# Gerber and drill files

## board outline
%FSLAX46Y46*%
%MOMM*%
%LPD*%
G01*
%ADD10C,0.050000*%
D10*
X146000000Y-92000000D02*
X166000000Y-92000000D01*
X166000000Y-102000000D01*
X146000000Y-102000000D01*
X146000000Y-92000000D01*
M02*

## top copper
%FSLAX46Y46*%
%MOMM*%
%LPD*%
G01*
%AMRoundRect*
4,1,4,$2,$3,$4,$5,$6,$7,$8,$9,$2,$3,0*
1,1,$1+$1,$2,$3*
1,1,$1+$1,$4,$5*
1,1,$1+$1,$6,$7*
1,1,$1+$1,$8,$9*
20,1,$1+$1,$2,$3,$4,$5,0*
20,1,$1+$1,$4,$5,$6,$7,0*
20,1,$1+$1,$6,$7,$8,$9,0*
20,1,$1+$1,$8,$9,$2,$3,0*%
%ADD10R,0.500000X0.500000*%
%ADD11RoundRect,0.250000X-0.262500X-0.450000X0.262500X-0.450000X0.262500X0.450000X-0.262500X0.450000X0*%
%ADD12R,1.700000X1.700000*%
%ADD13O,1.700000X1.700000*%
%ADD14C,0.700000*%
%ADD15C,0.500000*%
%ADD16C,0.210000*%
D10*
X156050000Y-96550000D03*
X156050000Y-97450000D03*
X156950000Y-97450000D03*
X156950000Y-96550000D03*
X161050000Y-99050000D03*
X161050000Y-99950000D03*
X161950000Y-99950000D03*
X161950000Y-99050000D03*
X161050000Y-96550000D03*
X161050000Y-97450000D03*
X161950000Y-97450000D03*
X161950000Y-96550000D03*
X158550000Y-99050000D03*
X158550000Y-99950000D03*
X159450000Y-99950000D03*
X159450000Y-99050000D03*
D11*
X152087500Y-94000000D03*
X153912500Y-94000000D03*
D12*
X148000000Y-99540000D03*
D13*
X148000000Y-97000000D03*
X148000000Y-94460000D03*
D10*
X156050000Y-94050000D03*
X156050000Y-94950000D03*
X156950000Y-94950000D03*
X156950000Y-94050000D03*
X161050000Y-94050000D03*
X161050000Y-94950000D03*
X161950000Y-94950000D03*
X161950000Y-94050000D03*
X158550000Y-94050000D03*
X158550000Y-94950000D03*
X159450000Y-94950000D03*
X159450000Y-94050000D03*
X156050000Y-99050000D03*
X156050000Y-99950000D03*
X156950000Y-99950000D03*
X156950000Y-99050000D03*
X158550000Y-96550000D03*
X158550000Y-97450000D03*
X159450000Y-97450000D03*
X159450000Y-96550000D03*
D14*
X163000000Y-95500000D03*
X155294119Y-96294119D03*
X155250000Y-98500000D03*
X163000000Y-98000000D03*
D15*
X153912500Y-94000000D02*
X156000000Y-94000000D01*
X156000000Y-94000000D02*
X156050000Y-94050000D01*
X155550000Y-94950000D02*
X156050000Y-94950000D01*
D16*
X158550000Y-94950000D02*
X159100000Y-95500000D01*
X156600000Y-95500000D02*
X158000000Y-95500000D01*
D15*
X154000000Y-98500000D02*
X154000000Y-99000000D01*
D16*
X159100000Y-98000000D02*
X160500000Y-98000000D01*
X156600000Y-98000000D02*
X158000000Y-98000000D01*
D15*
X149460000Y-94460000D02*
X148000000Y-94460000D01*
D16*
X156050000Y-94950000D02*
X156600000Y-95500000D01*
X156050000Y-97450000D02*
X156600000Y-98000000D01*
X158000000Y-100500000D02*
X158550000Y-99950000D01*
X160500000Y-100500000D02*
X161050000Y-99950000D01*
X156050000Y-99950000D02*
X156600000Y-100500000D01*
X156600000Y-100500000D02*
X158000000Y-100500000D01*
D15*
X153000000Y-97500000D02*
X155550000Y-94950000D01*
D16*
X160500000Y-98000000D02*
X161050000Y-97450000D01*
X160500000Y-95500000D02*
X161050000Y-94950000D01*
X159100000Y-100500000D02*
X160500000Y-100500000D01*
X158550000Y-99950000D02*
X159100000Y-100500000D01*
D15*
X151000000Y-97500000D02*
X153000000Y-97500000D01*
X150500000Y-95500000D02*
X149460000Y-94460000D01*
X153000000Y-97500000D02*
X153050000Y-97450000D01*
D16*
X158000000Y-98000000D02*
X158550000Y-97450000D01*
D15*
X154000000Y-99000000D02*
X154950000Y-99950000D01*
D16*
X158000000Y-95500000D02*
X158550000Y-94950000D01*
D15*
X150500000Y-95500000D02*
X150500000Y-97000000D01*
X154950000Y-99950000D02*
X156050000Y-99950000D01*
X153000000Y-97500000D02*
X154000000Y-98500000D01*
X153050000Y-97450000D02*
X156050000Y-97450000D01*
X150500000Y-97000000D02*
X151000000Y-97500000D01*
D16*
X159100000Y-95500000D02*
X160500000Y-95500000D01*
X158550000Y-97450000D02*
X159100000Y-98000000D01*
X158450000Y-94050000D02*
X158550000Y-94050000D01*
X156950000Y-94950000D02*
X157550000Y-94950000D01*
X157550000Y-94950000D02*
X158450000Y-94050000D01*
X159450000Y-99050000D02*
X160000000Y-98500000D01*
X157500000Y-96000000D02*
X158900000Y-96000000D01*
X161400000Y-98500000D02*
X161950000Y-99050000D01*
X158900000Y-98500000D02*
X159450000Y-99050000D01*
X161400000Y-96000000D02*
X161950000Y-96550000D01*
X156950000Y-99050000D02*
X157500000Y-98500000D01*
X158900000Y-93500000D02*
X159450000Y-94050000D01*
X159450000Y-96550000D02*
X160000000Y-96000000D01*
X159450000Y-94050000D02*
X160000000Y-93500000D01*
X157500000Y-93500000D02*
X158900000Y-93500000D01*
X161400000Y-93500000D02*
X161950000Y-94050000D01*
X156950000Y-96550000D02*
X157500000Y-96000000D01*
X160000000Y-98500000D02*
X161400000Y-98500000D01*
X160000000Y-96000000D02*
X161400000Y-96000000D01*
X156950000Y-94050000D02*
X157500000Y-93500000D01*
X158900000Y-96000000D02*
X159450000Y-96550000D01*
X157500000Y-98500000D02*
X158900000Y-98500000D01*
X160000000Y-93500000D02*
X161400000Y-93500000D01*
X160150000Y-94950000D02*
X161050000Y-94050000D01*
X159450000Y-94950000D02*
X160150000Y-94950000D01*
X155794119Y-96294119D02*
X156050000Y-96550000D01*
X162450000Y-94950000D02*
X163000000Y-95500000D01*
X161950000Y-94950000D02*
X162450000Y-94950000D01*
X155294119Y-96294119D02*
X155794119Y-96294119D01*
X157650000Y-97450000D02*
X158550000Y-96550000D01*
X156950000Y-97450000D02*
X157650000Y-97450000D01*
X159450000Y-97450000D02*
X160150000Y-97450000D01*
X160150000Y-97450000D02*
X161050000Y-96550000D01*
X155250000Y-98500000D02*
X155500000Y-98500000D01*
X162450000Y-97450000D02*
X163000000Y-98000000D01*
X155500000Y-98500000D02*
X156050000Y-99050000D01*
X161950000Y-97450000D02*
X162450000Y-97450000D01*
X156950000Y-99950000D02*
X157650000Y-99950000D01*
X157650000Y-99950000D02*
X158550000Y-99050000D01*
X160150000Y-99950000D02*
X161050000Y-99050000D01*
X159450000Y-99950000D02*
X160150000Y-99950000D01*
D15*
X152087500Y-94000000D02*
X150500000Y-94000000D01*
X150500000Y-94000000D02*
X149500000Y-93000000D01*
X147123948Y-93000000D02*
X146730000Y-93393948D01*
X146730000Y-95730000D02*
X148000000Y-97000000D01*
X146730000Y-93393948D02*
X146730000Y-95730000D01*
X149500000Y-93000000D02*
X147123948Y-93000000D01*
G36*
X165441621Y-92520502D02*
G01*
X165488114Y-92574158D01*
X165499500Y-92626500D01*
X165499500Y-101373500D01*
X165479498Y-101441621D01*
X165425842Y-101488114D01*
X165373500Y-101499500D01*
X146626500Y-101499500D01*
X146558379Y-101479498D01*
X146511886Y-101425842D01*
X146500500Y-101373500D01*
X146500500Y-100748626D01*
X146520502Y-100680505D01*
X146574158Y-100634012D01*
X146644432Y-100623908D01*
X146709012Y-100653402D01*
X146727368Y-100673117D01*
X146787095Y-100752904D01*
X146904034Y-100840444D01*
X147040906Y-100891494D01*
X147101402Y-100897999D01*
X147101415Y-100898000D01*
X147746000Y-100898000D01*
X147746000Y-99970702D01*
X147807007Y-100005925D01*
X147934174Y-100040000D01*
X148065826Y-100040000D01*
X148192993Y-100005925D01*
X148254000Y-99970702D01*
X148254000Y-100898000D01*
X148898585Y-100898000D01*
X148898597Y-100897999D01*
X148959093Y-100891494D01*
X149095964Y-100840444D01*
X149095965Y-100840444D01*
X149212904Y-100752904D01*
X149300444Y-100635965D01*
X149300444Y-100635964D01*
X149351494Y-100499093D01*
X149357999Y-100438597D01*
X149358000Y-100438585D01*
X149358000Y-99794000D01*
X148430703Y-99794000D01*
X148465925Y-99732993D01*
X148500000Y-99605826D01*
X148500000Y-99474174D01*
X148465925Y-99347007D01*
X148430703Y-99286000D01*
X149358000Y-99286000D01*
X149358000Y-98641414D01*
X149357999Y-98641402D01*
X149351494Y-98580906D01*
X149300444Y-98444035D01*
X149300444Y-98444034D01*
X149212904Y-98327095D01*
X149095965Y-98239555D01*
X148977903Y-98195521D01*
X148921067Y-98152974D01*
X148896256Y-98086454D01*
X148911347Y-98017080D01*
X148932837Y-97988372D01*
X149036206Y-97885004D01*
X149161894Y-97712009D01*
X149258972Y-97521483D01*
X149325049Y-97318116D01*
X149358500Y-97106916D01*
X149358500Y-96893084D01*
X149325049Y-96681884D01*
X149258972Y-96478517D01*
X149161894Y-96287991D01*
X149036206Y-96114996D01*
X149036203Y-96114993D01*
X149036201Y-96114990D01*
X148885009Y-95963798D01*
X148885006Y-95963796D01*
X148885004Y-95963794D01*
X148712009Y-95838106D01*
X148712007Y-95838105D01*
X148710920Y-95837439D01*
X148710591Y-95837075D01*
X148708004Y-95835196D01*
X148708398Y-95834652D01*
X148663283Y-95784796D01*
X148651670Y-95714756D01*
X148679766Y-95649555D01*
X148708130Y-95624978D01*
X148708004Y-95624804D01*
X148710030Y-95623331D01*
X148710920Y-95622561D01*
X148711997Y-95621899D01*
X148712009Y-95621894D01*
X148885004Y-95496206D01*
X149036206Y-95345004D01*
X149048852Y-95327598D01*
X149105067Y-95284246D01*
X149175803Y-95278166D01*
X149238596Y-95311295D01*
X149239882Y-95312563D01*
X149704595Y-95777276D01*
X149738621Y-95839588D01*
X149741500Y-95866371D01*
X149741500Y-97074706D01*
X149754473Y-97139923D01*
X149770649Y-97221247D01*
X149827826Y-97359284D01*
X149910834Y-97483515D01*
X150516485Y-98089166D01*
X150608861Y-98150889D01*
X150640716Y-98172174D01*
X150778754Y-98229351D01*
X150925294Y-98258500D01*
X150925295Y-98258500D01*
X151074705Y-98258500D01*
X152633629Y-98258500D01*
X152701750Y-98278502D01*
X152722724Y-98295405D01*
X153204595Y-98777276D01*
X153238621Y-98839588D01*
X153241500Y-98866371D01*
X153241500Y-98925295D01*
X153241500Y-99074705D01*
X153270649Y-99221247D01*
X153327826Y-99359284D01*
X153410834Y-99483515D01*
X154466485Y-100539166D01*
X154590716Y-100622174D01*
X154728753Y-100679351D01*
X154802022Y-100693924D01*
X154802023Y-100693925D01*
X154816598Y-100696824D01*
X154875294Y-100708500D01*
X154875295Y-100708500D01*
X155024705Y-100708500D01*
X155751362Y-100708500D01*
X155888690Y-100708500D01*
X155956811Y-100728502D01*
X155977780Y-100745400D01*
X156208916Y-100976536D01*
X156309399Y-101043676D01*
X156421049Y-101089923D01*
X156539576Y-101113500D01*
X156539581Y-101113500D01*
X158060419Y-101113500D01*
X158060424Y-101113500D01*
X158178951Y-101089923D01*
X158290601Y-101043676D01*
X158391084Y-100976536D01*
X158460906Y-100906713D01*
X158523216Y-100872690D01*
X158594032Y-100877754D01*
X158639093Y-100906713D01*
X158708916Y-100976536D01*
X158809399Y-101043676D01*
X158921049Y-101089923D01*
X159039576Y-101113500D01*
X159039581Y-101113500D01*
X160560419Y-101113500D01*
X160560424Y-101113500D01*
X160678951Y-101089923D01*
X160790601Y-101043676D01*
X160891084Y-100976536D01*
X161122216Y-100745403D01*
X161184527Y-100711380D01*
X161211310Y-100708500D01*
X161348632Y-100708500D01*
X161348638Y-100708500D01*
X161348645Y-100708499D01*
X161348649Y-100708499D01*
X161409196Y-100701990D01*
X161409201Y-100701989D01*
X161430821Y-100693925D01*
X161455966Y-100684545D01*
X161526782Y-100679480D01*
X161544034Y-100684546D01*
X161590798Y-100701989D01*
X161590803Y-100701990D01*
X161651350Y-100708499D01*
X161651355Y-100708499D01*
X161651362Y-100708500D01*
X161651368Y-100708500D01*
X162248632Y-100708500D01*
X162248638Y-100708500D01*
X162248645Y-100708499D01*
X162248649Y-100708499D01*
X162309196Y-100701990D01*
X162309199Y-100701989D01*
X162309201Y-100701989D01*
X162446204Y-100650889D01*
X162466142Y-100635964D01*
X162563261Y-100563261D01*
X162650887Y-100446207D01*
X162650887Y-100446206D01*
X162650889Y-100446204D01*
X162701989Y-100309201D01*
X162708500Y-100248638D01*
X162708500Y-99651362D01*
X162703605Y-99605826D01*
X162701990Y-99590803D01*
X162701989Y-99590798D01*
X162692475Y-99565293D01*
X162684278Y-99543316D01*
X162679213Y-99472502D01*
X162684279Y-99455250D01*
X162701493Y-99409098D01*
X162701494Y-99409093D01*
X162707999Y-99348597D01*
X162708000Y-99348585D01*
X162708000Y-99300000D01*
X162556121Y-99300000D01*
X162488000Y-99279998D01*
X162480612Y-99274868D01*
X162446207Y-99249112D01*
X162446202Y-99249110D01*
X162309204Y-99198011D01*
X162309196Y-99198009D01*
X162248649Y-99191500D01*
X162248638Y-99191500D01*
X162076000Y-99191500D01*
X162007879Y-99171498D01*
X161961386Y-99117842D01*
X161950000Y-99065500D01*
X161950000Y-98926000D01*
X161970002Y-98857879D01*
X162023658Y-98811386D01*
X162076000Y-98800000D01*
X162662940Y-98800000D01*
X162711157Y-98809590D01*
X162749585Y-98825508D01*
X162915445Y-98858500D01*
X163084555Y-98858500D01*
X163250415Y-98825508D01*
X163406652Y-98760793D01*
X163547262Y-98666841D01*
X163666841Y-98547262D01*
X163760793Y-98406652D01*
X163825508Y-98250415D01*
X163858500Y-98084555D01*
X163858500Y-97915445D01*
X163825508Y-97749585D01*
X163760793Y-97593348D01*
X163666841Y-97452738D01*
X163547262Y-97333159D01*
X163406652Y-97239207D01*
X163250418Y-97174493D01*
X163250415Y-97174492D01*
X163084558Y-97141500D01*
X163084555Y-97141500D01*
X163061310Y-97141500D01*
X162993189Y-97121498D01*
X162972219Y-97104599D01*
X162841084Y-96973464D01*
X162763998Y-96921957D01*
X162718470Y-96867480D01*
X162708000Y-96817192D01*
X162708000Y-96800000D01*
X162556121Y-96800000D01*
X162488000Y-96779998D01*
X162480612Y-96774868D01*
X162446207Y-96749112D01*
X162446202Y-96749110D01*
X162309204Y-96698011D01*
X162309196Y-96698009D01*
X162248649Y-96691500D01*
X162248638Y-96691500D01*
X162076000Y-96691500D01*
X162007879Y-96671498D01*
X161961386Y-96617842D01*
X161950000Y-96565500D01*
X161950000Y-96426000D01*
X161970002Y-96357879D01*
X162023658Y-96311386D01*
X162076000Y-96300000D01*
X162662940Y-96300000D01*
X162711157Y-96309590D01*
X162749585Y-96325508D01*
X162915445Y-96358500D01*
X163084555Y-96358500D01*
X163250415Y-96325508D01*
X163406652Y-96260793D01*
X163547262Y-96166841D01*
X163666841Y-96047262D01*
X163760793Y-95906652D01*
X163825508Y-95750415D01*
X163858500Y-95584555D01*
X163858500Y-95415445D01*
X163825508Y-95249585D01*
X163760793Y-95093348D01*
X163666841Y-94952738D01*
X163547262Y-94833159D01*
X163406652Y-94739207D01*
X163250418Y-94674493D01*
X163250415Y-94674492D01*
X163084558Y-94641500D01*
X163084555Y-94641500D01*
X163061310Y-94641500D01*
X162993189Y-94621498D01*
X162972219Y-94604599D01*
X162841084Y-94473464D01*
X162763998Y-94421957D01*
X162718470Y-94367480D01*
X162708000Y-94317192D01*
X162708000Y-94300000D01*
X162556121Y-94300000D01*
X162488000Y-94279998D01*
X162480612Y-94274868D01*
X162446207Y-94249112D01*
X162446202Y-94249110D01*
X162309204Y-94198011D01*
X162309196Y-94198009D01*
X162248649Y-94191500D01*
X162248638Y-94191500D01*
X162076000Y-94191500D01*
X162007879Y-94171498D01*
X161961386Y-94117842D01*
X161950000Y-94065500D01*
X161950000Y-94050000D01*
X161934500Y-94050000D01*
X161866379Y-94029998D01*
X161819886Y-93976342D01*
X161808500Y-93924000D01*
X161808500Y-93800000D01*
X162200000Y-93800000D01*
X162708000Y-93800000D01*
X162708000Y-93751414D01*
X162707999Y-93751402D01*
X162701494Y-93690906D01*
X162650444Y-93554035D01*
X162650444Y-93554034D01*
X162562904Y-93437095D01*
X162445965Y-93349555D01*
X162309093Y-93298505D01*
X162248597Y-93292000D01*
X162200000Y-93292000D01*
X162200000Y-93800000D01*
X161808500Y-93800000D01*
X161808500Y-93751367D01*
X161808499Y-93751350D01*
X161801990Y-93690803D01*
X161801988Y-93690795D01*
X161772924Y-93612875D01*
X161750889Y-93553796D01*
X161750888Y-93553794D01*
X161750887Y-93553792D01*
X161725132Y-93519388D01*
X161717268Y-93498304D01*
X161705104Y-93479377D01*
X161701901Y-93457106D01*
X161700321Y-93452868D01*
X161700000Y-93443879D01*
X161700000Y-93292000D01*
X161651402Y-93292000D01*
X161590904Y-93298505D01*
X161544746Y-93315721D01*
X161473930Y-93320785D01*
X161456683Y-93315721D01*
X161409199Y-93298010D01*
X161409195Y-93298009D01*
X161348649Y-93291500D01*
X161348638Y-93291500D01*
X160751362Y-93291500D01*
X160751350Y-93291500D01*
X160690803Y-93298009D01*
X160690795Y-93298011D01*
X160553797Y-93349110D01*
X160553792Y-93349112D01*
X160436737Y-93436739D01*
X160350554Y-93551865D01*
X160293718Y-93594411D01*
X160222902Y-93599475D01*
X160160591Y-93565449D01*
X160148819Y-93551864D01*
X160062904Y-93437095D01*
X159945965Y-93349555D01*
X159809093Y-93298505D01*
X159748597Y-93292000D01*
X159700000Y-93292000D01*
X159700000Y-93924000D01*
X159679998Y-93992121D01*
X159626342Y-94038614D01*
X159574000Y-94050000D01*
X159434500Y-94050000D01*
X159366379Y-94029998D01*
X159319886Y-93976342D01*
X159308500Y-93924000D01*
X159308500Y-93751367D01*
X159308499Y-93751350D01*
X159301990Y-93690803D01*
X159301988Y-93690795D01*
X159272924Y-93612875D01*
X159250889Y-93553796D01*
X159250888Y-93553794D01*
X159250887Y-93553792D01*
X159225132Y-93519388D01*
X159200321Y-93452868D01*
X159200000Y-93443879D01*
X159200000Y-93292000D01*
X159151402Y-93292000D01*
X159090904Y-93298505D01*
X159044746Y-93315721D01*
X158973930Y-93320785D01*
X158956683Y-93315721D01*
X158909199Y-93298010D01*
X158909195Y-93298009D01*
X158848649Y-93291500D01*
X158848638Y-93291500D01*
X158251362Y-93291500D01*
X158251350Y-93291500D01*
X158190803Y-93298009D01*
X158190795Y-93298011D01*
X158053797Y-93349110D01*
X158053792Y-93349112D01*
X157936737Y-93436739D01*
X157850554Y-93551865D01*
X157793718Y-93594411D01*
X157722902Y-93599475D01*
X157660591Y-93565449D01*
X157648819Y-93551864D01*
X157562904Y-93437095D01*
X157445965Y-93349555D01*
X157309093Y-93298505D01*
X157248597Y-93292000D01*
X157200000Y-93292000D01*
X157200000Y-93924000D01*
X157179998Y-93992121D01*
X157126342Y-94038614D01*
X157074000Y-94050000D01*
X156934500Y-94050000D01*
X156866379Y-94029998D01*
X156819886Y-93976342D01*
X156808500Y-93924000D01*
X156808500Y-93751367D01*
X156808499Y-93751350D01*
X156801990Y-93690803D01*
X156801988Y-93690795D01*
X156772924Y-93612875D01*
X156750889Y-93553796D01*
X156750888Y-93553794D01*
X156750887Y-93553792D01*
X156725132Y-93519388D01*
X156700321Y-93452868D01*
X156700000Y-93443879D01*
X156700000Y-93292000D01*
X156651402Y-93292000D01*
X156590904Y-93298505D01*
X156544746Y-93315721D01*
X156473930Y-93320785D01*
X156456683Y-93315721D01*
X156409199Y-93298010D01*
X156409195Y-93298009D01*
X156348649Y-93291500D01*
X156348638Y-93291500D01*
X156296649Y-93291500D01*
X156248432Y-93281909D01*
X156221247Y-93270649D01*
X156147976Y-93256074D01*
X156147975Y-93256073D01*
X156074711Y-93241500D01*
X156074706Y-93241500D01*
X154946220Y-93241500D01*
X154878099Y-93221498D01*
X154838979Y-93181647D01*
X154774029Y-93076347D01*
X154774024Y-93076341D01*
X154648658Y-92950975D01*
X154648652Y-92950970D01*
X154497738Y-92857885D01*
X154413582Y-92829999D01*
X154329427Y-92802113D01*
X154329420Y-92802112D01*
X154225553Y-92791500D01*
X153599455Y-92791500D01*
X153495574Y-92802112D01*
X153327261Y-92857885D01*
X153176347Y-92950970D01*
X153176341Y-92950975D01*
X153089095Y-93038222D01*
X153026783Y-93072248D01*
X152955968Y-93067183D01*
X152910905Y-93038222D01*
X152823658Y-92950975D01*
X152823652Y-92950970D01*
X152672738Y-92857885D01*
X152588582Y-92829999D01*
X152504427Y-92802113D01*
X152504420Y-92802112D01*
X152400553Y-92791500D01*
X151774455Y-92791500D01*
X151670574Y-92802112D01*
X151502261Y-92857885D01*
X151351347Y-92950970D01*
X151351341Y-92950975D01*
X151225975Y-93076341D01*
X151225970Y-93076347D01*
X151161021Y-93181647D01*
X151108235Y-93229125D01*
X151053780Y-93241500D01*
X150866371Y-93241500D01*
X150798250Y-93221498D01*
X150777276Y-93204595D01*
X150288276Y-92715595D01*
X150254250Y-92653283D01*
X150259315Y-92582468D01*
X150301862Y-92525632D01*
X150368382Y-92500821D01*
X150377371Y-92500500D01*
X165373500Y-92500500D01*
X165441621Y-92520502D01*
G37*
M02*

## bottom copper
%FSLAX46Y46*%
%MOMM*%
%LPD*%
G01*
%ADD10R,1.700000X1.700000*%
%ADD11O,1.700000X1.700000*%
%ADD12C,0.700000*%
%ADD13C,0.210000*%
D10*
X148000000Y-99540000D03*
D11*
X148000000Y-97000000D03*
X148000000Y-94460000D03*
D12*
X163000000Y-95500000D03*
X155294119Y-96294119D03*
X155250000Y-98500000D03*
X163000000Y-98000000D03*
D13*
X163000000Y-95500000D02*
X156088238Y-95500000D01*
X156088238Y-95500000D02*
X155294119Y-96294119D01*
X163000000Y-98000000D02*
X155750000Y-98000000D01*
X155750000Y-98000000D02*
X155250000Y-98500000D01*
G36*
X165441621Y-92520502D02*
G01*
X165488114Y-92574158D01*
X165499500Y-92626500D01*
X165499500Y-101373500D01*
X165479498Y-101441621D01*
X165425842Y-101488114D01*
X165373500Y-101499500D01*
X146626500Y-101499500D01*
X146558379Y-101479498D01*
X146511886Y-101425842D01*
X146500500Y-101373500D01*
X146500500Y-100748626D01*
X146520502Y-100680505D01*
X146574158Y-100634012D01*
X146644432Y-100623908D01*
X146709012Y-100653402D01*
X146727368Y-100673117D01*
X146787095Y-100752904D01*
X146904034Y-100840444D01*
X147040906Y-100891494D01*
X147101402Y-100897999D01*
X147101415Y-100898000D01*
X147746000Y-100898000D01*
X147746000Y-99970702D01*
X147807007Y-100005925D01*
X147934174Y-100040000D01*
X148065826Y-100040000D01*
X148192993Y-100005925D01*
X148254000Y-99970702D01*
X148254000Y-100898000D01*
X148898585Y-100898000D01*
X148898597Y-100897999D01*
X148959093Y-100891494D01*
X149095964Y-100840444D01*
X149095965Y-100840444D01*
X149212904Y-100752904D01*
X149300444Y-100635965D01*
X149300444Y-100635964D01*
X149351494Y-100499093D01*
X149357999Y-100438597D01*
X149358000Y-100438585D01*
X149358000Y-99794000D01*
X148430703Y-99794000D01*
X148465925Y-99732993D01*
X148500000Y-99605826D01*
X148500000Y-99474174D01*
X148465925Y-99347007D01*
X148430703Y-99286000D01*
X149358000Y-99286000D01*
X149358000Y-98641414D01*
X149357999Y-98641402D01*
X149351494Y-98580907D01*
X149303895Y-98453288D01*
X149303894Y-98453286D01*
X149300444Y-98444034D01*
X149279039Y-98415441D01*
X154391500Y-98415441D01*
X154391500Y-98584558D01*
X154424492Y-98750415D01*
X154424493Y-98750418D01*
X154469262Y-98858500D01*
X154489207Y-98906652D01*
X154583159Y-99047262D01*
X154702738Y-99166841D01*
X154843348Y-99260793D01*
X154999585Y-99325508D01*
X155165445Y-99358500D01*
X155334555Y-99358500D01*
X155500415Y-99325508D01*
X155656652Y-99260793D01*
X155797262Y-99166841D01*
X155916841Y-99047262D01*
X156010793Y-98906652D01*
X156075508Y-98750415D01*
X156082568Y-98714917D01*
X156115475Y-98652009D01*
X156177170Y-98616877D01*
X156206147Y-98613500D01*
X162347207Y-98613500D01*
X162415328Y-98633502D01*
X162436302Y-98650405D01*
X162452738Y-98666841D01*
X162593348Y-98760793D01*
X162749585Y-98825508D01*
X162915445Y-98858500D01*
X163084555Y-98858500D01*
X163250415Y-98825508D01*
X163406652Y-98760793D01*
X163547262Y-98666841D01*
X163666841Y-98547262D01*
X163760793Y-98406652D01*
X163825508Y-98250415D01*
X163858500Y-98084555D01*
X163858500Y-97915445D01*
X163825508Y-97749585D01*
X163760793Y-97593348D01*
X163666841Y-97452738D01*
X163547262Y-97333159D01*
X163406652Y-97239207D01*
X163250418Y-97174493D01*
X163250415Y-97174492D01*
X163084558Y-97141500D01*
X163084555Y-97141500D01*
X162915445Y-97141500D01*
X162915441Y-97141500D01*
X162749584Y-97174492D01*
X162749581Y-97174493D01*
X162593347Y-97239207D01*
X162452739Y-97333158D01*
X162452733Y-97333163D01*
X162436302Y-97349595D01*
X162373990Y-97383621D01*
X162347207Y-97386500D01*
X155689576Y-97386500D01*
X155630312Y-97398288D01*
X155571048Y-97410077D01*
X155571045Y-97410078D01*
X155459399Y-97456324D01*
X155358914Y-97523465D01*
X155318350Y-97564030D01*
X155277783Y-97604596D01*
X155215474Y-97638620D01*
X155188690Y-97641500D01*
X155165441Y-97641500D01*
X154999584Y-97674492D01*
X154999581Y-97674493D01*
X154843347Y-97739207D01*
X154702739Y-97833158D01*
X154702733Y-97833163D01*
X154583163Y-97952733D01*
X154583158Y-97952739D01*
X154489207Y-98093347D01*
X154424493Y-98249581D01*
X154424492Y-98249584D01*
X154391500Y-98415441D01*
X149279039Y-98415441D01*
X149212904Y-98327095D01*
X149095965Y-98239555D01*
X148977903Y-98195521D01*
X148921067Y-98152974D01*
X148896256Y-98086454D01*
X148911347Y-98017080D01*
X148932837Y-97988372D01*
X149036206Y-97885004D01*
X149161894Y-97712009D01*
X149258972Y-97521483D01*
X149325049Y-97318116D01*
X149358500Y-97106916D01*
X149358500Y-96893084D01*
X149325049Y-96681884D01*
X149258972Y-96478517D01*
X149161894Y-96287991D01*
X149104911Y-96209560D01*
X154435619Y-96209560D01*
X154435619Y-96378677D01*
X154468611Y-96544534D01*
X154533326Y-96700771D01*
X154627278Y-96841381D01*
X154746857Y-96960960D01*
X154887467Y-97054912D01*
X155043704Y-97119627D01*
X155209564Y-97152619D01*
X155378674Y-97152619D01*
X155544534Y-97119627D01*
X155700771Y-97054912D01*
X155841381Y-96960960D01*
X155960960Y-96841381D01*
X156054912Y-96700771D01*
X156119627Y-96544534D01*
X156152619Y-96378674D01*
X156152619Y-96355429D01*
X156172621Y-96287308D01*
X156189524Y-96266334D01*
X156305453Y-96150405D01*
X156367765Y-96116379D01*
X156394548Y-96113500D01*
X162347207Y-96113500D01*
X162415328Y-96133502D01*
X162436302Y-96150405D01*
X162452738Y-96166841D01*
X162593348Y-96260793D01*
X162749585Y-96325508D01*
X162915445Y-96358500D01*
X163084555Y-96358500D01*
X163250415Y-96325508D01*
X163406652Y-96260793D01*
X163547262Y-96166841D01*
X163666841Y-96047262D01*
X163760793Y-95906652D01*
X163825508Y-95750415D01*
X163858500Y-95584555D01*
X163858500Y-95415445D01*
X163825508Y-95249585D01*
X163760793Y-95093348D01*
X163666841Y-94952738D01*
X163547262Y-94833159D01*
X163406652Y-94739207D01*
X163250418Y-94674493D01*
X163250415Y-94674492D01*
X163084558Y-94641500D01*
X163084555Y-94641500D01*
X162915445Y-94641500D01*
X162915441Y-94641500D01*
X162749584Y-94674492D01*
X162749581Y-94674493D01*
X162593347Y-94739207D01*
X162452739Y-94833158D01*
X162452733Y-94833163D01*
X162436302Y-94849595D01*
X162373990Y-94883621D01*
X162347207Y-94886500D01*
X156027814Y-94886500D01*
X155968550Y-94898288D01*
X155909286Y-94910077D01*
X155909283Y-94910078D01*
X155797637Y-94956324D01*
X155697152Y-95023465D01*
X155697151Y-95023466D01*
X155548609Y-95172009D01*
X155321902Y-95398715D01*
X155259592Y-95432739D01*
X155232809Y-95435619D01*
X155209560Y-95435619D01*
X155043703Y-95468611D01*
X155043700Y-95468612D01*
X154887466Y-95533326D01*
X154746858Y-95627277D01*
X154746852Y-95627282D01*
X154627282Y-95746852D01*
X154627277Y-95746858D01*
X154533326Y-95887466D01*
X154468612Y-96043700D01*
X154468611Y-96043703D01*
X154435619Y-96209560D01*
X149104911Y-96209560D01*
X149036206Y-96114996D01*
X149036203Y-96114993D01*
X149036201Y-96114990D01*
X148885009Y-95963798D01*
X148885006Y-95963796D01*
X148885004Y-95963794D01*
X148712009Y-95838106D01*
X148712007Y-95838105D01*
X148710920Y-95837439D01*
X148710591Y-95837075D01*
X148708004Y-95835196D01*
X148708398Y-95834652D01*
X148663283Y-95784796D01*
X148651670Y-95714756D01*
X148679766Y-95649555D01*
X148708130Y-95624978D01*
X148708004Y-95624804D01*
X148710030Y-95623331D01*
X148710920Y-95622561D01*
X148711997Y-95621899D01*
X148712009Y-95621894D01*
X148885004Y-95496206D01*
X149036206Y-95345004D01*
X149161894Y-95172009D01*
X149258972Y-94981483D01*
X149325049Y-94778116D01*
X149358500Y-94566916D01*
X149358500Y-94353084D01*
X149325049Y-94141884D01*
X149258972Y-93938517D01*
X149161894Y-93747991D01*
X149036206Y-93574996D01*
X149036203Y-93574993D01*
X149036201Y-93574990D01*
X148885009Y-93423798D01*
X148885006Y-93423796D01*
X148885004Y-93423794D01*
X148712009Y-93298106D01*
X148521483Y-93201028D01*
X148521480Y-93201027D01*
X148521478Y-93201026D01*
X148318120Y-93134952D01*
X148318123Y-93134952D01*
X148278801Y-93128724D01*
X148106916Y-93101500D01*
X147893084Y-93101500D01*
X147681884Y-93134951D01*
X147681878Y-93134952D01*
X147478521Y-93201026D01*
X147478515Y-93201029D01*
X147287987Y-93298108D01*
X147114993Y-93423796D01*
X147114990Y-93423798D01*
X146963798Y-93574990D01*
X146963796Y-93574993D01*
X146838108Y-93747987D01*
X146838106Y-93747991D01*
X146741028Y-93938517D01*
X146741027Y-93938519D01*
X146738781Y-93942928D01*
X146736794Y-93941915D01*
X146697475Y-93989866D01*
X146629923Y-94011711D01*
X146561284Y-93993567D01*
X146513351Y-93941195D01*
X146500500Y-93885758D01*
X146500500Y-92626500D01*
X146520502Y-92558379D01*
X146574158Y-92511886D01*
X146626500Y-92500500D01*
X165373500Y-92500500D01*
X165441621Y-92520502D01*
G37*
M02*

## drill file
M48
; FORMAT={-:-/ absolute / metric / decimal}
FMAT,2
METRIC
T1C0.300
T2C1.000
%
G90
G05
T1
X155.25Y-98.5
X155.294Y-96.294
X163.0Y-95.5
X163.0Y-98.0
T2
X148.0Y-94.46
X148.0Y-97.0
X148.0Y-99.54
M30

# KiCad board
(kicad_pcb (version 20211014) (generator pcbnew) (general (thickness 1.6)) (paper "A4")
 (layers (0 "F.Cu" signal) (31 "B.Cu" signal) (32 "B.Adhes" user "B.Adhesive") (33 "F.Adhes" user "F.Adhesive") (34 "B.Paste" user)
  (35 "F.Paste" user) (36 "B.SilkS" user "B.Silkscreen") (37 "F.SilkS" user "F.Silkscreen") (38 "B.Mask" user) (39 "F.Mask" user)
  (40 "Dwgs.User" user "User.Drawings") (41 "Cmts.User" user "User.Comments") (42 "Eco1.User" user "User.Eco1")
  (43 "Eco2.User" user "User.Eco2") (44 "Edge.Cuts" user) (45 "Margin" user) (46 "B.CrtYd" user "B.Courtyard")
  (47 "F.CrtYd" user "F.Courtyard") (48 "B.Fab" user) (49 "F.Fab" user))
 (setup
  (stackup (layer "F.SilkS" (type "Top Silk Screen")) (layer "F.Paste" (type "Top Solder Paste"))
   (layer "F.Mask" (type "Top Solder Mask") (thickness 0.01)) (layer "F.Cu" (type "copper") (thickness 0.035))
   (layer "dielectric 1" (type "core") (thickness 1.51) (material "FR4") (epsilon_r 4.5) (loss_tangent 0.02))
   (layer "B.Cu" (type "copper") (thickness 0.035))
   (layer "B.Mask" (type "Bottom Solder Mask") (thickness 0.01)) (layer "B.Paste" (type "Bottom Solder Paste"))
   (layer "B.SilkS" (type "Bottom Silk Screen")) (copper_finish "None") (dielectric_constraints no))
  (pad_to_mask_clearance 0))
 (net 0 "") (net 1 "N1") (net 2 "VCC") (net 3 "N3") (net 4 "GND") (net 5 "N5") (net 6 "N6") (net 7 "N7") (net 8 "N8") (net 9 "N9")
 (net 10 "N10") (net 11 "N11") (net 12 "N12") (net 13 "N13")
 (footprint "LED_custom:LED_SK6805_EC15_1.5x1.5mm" (layer "F.Cu") (at 156.5 97)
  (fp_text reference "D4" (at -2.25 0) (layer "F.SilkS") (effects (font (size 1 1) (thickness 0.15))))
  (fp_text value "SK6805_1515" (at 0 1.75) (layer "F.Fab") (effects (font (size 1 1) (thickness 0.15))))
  (pad "1" smd rect (at -0.45 -0.45) (size 0.5 0.5) (layers "F.Cu" "F.Paste" "F.Mask") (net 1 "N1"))
  (pad "2" smd rect (at -0.45 0.45) (size 0.5 0.5) (layers "F.Cu" "F.Paste" "F.Mask") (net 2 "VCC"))
  (pad "3" smd rect (at 0.45 0.45) (size 0.5 0.5) (layers "F.Cu" "F.Paste" "F.Mask") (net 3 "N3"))
  (pad "4" smd rect (at 0.45 -0.45) (size 0.5 0.5) (layers "F.Cu" "F.Paste" "F.Mask") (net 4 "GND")))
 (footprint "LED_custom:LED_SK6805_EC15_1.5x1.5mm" (layer "F.Cu") (at 161.5 99.5)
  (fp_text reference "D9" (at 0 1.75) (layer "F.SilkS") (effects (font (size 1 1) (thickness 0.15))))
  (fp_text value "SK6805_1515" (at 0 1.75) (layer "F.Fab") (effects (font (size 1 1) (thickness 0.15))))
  (pad "1" smd rect (at -0.45 -0.45) (size 0.5 0.5) (layers "F.Cu" "F.Paste" "F.Mask") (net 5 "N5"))
  (pad "2" smd rect (at -0.45 0.45) (size 0.5 0.5) (layers "F.Cu" "F.Paste" "F.Mask") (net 2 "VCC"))
  (pad "3" smd rect (at 0.45 0.45) (size 0.5 0.5) (layers "F.Cu" "F.Paste" "F.Mask") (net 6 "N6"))
  (pad "4" smd rect (at 0.45 -0.45) (size 0.5 0.5) (layers "F.Cu" "F.Paste" "F.Mask") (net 4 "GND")))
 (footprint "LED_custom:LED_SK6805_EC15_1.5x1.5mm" (layer "F.Cu") (at 161.5 97)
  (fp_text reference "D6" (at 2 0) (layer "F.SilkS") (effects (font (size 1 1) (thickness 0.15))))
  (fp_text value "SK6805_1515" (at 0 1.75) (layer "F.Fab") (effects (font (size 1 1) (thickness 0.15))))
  (pad "1" smd rect (at -0.45 -0.45) (size 0.5 0.5) (layers "F.Cu" "F.Paste" "F.Mask") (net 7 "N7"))
  (pad "2" smd rect (at -0.45 0.45) (size 0.5 0.5) (layers "F.Cu" "F.Paste" "F.Mask") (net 2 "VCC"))
  (pad "3" smd rect (at 0.45 0.45) (size 0.5 0.5) (layers "F.Cu" "F.Paste" "F.Mask") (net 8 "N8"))
  (pad "4" smd rect (at 0.45 -0.45) (size 0.5 0.5) (layers "F.Cu" "F.Paste" "F.Mask") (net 4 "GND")))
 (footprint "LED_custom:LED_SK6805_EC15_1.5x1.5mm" (layer "F.Cu") (at 159 99.5)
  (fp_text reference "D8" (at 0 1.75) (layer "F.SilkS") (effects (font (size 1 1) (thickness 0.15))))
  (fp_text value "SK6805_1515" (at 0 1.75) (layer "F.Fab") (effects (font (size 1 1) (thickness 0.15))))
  (pad "1" smd rect (at -0.45 -0.45) (size 0.5 0.5) (layers "F.Cu" "F.Paste" "F.Mask") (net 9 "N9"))
  (pad "2" smd rect (at -0.45 0.45) (size 0.5 0.5) (layers "F.Cu" "F.Paste" "F.Mask") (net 2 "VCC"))
  (pad "3" smd rect (at 0.45 0.45) (size 0.5 0.5) (layers "F.Cu" "F.Paste" "F.Mask") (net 5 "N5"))
  (pad "4" smd rect (at 0.45 -0.45) (size 0.5 0.5) (layers "F.Cu" "F.Paste" "F.Mask") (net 4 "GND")))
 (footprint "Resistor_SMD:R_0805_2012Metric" (layer "F.Cu") (at 153 94)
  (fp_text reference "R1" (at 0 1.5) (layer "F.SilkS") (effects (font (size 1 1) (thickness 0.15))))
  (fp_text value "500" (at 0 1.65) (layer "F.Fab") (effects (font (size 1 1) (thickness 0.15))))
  (pad "1" smd roundrect (at -0.9125 0) (size 1.025 1.4) (layers "F.Cu" "F.Paste" "F.Mask") (roundrect_rratio 0.243902) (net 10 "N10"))
  (pad "2" smd roundrect (at 0.9125 0) (size 1.025 1.4) (layers "F.Cu" "F.Paste" "F.Mask") (roundrect_rratio 0.243902) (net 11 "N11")))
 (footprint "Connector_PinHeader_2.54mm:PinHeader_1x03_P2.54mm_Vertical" (layer "F.Cu") (at 148 99.54 180)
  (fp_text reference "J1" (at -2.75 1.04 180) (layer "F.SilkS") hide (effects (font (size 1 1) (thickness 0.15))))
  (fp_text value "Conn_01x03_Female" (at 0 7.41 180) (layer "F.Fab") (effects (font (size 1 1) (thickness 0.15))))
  (pad "1" thru_hole rect (at 0 0 180) (size 1.7 1.7) (drill 1) (layers *.Cu *.Mask) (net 4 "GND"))
  (pad "2" thru_hole oval (at 0 2.54 180) (size 1.7 1.7) (drill 1) (layers *.Cu *.Mask) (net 10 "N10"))
  (pad "3" thru_hole oval (at 0 5.08 180) (size 1.7 1.7) (drill 1) (layers *.Cu *.Mask) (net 2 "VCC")))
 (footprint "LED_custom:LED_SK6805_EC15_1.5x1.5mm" (layer "F.Cu") (at 156.5 94.5)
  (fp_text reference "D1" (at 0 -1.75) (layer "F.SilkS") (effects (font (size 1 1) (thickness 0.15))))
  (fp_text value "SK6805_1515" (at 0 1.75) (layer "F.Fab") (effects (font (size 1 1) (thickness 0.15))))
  (pad "1" smd rect (at -0.45 -0.45) (size 0.5 0.5) (layers "F.Cu" "F.Paste" "F.Mask") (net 11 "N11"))
  (pad "2" smd rect (at -0.45 0.45) (size 0.5 0.5) (layers "F.Cu" "F.Paste" "F.Mask") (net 2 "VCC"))
  (pad "3" smd rect (at 0.45 0.45) (size 0.5 0.5) (layers "F.Cu" "F.Paste" "F.Mask") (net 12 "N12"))
  (pad "4" smd rect (at 0.45 -0.45) (size 0.5 0.5) (layers "F.Cu" "F.Paste" "F.Mask") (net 4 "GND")))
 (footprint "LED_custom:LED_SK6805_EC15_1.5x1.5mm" (layer "F.Cu") (at 161.5 94.5)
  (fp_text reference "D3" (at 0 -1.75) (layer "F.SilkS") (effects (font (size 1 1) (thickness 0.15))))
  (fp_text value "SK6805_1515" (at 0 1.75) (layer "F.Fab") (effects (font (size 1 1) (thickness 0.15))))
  (pad "1" smd rect (at -0.45 -0.45) (size 0.5 0.5) (layers "F.Cu" "F.Paste" "F.Mask") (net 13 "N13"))
  (pad "2" smd rect (at -0.45 0.45) (size 0.5 0.5) (layers "F.Cu" "F.Paste" "F.Mask") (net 2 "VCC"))
  (pad "3" smd rect (at 0.45 0.45) (size 0.5 0.5) (layers "F.Cu" "F.Paste" "F.Mask") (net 1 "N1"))
  (pad "4" smd rect (at 0.45 -0.45) (size 0.5 0.5) (layers "F.Cu" "F.Paste" "F.Mask") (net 4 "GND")))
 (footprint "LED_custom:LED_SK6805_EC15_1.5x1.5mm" (layer "F.Cu") (at 159 94.5)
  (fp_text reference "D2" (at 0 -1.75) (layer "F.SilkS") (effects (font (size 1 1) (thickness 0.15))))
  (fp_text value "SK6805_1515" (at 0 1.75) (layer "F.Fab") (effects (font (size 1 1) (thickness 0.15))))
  (pad "1" smd rect (at -0.45 -0.45) (size 0.5 0.5) (layers "F.Cu" "F.Paste" "F.Mask") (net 12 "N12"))
  (pad "2" smd rect (at -0.45 0.45) (size 0.5 0.5) (layers "F.Cu" "F.Paste" "F.Mask") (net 2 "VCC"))
  (pad "3" smd rect (at 0.45 0.45) (size 0.5 0.5) (layers "F.Cu" "F.Paste" "F.Mask") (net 13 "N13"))
  (pad "4" smd rect (at 0.45 -0.45) (size 0.5 0.5) (layers "F.Cu" "F.Paste" "F.Mask") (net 4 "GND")))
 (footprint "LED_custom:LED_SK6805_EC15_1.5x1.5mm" (layer "F.Cu") (at 156.5 99.5)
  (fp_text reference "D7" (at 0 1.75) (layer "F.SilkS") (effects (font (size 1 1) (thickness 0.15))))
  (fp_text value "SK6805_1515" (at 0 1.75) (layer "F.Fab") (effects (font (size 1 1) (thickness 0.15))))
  (pad "1" smd rect (at -0.45 -0.45) (size 0.5 0.5) (layers "F.Cu" "F.Paste" "F.Mask") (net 8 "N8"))
  (pad "2" smd rect (at -0.45 0.45) (size 0.5 0.5) (layers "F.Cu" "F.Paste" "F.Mask") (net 2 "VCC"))
  (pad "3" smd rect (at 0.45 0.45) (size 0.5 0.5) (layers "F.Cu" "F.Paste" "F.Mask") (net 9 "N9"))
  (pad "4" smd rect (at 0.45 -0.45) (size 0.5 0.5) (layers "F.Cu" "F.Paste" "F.Mask") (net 4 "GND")))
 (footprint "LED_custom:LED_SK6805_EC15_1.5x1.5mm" (layer "F.Cu") (at 159 97)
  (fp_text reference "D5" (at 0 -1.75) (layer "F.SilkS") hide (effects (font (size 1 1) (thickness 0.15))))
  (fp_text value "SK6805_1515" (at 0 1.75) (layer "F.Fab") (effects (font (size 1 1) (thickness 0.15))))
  (pad "1" smd rect (at -0.45 -0.45) (size 0.5 0.5) (layers "F.Cu" "F.Paste" "F.Mask") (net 3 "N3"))
  (pad "2" smd rect (at -0.45 0.45) (size 0.5 0.5) (layers "F.Cu" "F.Paste" "F.Mask") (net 2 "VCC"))
  (pad "3" smd rect (at 0.45 0.45) (size 0.5 0.5) (layers "F.Cu" "F.Paste" "F.Mask") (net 7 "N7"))
  (pad "4" smd rect (at 0.45 -0.45) (size 0.5 0.5) (layers "F.Cu" "F.Paste" "F.Mask") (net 4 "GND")))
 (gr_rect (start 146 92) (end 166 102) (layer "Edge.Cuts") (width 0.05) (fill none))
 (segment (start 153.9125 94) (end 156 94) (width 0.5) (layer "F.Cu") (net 11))
 (segment (start 156 94) (end 156.05 94.05) (width 0.5) (layer "F.Cu") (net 11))
 (segment (start 155.55 94.95) (end 156.05 94.95) (width 0.5) (layer "F.Cu") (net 2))
 (segment (start 158.55 94.95) (end 159.1 95.5) (width 0.21) (layer "F.Cu") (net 2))
 (segment (start 156.6 95.5) (end 158 95.5) (width 0.21) (layer "F.Cu") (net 2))
 (segment (start 154 98.5) (end 154 99) (width 0.5) (layer "F.Cu") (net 2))
 (segment (start 159.1 98) (end 160.5 98) (width 0.21) (layer "F.Cu") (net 2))
 (segment (start 156.6 98) (end 158 98) (width 0.21) (layer "F.Cu") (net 2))
 (segment (start 149.46 94.46) (end 148 94.46) (width 0.5) (layer "F.Cu") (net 2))
 (segment (start 156.05 94.95) (end 156.6 95.5) (width 0.21) (layer "F.Cu") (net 2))
 (segment (start 156.05 97.45) (end 156.6 98) (width 0.21) (layer "F.Cu") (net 2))
 (segment (start 158 100.5) (end 158.55 99.95) (width 0.21) (layer "F.Cu") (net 2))
 (segment (start 160.5 100.5) (end 161.05 99.95) (width 0.21) (layer "F.Cu") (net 2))
 (segment (start 156.05 99.95) (end 156.6 100.5) (width 0.21) (layer "F.Cu") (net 2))
 (segment (start 156.6 100.5) (end 158 100.5) (width 0.21) (layer "F.Cu") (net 2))
 (segment (start 153 97.5) (end 155.55 94.95) (width 0.5) (layer "F.Cu") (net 2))
 (segment (start 160.5 98) (end 161.05 97.45) (width 0.21) (layer "F.Cu") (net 2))
 (segment (start 160.5 95.5) (end 161.05 94.95) (width 0.21) (layer "F.Cu") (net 2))
 (segment (start 159.1 100.5) (end 160.5 100.5) (width 0.21) (layer "F.Cu") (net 2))
 (segment (start 158.55 99.95) (end 159.1 100.5) (width 0.21) (layer "F.Cu") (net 2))
 (segment (start 151 97.5) (end 153 97.5) (width 0.5) (layer "F.Cu") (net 2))
 (segment (start 150.5 95.5) (end 149.46 94.46) (width 0.5) (layer "F.Cu") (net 2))
 (segment (start 153 97.5) (end 153.05 97.45) (width 0.5) (layer "F.Cu") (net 2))
 (segment (start 158 98) (end 158.55 97.45) (width 0.21) (layer "F.Cu") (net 2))
 (segment (start 154 99) (end 154.95 99.95) (width 0.5) (layer "F.Cu") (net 2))
 (segment (start 158 95.5) (end 158.55 94.95) (width 0.21) (layer "F.Cu") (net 2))
 (segment (start 150.5 95.5) (end 150.5 97) (width 0.5) (layer "F.Cu") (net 2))
 (segment (start 154.95 99.95) (end 156.05 99.95) (width 0.5) (layer "F.Cu") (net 2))
 (segment (start 153 97.5) (end 154 98.5) (width 0.5) (layer "F.Cu") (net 2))
 (segment (start 153.05 97.45) (end 156.05 97.45) (width 0.5) (layer "F.Cu") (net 2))
 (segment (start 150.5 97) (end 151 97.5) (width 0.5) (layer "F.Cu") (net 2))
 (segment (start 159.1 95.5) (end 160.5 95.5) (width 0.21) (layer "F.Cu") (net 2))
 (segment (start 158.55 97.45) (end 159.1 98) (width 0.21) (layer "F.Cu") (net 2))
 (segment (start 158.45 94.05) (end 158.55 94.05) (width 0.21) (layer "F.Cu") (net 12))
 (segment (start 156.95 94.95) (end 157.55 94.95) (width 0.21) (layer "F.Cu") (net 12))
 (segment (start 157.55 94.95) (end 158.45 94.05) (width 0.21) (layer "F.Cu") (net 12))
 (segment (start 159.45 99.05) (end 160 98.5) (width 0.21) (layer "F.Cu") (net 4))
 (segment (start 157.5 96) (end 158.9 96) (width 0.21) (layer "F.Cu") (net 4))
 (segment (start 161.4 98.5) (end 161.95 99.05) (width 0.21) (layer "F.Cu") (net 4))
 (segment (start 158.9 98.5) (end 159.45 99.05) (width 0.21) (layer "F.Cu") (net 4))
 (segment (start 161.4 96) (end 161.95 96.55) (width 0.21) (layer "F.Cu") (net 4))
 (segment (start 156.95 99.05) (end 157.5 98.5) (width 0.21) (layer "F.Cu") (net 4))
 (segment (start 158.9 93.5) (end 159.45 94.05) (width 0.21) (layer "F.Cu") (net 4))
 (segment (start 159.45 96.55) (end 160 96) (width 0.21) (layer "F.Cu") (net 4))
 (segment (start 159.45 94.05) (end 160 93.5) (width 0.21) (layer "F.Cu") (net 4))
 (segment (start 157.5 93.5) (end 158.9 93.5) (width 0.21) (layer "F.Cu") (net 4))
 (segment (start 161.4 93.5) (end 161.95 94.05) (width 0.21) (layer "F.Cu") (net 4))
 (segment (start 156.95 96.55) (end 157.5 96) (width 0.21) (layer "F.Cu") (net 4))
 (segment (start 160 98.5) (end 161.4 98.5) (width 0.21) (layer "F.Cu") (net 4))
 (segment (start 160 96) (end 161.4 96) (width 0.21) (layer "F.Cu") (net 4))
 (segment (start 156.95 94.05) (end 157.5 93.5) (width 0.21) (layer "F.Cu") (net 4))
 (segment (start 158.9 96) (end 159.45 96.55) (width 0.21) (layer "F.Cu") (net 4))
 (segment (start 157.5 98.5) (end 158.9 98.5) (width 0.21) (layer "F.Cu") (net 4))
 (segment (start 160 93.5) (end 161.4 93.5) (width 0.21) (layer "F.Cu") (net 4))
 (segment (start 160.15 94.95) (end 161.05 94.05) (width 0.21) (layer "F.Cu") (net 13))
 (segment (start 159.45 94.95) (end 160.15 94.95) (width 0.21) (layer "F.Cu") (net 13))
 (segment (start 155.794119 96.294119) (end 156.05 96.55) (width 0.21) (layer "F.Cu") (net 1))
 (segment (start 162.45 94.95) (end 163 95.5) (width 0.21) (layer "F.Cu") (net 1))
 (segment (start 161.95 94.95) (end 162.45 94.95) (width 0.21) (layer "F.Cu") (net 1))
 (segment (start 155.294119 96.294119) (end 155.794119 96.294119) (width 0.21) (layer "F.Cu") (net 1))
 (via (at 163 95.5) (size 0.7) (drill 0.3) (layers "F.Cu" "B.Cu") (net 1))
 (via (at 155.294119 96.294119) (size 0.7) (drill 0.3) (layers "F.Cu" "B.Cu") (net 1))
 (segment (start 163 95.5) (end 156.088238 95.5) (width 0.21) (layer "B.Cu") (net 1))
 (segment (start 156.088238 95.5) (end 155.294119 96.294119) (width 0.21) (layer "B.Cu") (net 1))
 (segment (start 157.65 97.45) (end 158.55 96.55) (width 0.21) (layer "F.Cu") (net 3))
 (segment (start 156.95 97.45) (end 157.65 97.45) (width 0.21) (layer "F.Cu") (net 3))
 (segment (start 159.45 97.45) (end 160.15 97.45) (width 0.21) (layer "F.Cu") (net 7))
 (segment (start 160.15 97.45) (end 161.05 96.55) (width 0.21) (layer "F.Cu") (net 7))
 (segment (start 155.25 98.5) (end 155.5 98.5) (width 0.21) (layer "F.Cu") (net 8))
 (segment (start 162.45 97.45) (end 163 98) (width 0.21) (layer "F.Cu") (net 8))
 (segment (start 155.5 98.5) (end 156.05 99.05) (width 0.21) (layer "F.Cu") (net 8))
 (segment (start 161.95 97.45) (end 162.45 97.45) (width 0.21) (layer "F.Cu") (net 8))
 (via (at 155.25 98.5) (size 0.7) (drill 0.3) (layers "F.Cu" "B.Cu") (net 8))
 (via (at 163 98) (size 0.7) (drill 0.3) (layers "F.Cu" "B.Cu") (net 8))
 (segment (start 163 98) (end 155.75 98) (width 0.21) (layer "B.Cu") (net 8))
 (segment (start 155.75 98) (end 155.25 98.5) (width 0.21) (layer "B.Cu") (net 8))
 (segment (start 156.95 99.95) (end 157.65 99.95) (width 0.21) (layer "F.Cu") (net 9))
 (segment (start 157.65 99.95) (end 158.55 99.05) (width 0.21) (layer "F.Cu") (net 9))
 (segment (start 160.15 99.95) (end 161.05 99.05) (width 0.21) (layer "F.Cu") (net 5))
 (segment (start 159.45 99.95) (end 160.15 99.95) (width 0.21) (layer "F.Cu") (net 5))
 (segment (start 152.0875 94) (end 150.5 94) (width 0.5) (layer "F.Cu") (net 10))
 (segment (start 150.5 94) (end 149.5 93) (width 0.5) (layer "F.Cu") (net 10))
 (segment (start 147.123948 93) (end 146.73 93.393948) (width 0.5) (layer "F.Cu") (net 10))
 (segment (start 146.73 95.73) (end 148 97) (width 0.5) (layer "F.Cu") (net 10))
 (segment (start 146.73 93.393948) (end 146.73 95.73) (width 0.5) (layer "F.Cu") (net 10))
 (segment (start 149.5 93) (end 147.123948 93) (width 0.5) (layer "F.Cu") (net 10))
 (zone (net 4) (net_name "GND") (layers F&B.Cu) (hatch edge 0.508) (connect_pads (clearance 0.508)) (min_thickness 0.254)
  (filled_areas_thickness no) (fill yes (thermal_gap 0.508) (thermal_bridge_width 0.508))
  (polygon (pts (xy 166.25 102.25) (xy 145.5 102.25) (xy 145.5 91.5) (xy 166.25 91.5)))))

